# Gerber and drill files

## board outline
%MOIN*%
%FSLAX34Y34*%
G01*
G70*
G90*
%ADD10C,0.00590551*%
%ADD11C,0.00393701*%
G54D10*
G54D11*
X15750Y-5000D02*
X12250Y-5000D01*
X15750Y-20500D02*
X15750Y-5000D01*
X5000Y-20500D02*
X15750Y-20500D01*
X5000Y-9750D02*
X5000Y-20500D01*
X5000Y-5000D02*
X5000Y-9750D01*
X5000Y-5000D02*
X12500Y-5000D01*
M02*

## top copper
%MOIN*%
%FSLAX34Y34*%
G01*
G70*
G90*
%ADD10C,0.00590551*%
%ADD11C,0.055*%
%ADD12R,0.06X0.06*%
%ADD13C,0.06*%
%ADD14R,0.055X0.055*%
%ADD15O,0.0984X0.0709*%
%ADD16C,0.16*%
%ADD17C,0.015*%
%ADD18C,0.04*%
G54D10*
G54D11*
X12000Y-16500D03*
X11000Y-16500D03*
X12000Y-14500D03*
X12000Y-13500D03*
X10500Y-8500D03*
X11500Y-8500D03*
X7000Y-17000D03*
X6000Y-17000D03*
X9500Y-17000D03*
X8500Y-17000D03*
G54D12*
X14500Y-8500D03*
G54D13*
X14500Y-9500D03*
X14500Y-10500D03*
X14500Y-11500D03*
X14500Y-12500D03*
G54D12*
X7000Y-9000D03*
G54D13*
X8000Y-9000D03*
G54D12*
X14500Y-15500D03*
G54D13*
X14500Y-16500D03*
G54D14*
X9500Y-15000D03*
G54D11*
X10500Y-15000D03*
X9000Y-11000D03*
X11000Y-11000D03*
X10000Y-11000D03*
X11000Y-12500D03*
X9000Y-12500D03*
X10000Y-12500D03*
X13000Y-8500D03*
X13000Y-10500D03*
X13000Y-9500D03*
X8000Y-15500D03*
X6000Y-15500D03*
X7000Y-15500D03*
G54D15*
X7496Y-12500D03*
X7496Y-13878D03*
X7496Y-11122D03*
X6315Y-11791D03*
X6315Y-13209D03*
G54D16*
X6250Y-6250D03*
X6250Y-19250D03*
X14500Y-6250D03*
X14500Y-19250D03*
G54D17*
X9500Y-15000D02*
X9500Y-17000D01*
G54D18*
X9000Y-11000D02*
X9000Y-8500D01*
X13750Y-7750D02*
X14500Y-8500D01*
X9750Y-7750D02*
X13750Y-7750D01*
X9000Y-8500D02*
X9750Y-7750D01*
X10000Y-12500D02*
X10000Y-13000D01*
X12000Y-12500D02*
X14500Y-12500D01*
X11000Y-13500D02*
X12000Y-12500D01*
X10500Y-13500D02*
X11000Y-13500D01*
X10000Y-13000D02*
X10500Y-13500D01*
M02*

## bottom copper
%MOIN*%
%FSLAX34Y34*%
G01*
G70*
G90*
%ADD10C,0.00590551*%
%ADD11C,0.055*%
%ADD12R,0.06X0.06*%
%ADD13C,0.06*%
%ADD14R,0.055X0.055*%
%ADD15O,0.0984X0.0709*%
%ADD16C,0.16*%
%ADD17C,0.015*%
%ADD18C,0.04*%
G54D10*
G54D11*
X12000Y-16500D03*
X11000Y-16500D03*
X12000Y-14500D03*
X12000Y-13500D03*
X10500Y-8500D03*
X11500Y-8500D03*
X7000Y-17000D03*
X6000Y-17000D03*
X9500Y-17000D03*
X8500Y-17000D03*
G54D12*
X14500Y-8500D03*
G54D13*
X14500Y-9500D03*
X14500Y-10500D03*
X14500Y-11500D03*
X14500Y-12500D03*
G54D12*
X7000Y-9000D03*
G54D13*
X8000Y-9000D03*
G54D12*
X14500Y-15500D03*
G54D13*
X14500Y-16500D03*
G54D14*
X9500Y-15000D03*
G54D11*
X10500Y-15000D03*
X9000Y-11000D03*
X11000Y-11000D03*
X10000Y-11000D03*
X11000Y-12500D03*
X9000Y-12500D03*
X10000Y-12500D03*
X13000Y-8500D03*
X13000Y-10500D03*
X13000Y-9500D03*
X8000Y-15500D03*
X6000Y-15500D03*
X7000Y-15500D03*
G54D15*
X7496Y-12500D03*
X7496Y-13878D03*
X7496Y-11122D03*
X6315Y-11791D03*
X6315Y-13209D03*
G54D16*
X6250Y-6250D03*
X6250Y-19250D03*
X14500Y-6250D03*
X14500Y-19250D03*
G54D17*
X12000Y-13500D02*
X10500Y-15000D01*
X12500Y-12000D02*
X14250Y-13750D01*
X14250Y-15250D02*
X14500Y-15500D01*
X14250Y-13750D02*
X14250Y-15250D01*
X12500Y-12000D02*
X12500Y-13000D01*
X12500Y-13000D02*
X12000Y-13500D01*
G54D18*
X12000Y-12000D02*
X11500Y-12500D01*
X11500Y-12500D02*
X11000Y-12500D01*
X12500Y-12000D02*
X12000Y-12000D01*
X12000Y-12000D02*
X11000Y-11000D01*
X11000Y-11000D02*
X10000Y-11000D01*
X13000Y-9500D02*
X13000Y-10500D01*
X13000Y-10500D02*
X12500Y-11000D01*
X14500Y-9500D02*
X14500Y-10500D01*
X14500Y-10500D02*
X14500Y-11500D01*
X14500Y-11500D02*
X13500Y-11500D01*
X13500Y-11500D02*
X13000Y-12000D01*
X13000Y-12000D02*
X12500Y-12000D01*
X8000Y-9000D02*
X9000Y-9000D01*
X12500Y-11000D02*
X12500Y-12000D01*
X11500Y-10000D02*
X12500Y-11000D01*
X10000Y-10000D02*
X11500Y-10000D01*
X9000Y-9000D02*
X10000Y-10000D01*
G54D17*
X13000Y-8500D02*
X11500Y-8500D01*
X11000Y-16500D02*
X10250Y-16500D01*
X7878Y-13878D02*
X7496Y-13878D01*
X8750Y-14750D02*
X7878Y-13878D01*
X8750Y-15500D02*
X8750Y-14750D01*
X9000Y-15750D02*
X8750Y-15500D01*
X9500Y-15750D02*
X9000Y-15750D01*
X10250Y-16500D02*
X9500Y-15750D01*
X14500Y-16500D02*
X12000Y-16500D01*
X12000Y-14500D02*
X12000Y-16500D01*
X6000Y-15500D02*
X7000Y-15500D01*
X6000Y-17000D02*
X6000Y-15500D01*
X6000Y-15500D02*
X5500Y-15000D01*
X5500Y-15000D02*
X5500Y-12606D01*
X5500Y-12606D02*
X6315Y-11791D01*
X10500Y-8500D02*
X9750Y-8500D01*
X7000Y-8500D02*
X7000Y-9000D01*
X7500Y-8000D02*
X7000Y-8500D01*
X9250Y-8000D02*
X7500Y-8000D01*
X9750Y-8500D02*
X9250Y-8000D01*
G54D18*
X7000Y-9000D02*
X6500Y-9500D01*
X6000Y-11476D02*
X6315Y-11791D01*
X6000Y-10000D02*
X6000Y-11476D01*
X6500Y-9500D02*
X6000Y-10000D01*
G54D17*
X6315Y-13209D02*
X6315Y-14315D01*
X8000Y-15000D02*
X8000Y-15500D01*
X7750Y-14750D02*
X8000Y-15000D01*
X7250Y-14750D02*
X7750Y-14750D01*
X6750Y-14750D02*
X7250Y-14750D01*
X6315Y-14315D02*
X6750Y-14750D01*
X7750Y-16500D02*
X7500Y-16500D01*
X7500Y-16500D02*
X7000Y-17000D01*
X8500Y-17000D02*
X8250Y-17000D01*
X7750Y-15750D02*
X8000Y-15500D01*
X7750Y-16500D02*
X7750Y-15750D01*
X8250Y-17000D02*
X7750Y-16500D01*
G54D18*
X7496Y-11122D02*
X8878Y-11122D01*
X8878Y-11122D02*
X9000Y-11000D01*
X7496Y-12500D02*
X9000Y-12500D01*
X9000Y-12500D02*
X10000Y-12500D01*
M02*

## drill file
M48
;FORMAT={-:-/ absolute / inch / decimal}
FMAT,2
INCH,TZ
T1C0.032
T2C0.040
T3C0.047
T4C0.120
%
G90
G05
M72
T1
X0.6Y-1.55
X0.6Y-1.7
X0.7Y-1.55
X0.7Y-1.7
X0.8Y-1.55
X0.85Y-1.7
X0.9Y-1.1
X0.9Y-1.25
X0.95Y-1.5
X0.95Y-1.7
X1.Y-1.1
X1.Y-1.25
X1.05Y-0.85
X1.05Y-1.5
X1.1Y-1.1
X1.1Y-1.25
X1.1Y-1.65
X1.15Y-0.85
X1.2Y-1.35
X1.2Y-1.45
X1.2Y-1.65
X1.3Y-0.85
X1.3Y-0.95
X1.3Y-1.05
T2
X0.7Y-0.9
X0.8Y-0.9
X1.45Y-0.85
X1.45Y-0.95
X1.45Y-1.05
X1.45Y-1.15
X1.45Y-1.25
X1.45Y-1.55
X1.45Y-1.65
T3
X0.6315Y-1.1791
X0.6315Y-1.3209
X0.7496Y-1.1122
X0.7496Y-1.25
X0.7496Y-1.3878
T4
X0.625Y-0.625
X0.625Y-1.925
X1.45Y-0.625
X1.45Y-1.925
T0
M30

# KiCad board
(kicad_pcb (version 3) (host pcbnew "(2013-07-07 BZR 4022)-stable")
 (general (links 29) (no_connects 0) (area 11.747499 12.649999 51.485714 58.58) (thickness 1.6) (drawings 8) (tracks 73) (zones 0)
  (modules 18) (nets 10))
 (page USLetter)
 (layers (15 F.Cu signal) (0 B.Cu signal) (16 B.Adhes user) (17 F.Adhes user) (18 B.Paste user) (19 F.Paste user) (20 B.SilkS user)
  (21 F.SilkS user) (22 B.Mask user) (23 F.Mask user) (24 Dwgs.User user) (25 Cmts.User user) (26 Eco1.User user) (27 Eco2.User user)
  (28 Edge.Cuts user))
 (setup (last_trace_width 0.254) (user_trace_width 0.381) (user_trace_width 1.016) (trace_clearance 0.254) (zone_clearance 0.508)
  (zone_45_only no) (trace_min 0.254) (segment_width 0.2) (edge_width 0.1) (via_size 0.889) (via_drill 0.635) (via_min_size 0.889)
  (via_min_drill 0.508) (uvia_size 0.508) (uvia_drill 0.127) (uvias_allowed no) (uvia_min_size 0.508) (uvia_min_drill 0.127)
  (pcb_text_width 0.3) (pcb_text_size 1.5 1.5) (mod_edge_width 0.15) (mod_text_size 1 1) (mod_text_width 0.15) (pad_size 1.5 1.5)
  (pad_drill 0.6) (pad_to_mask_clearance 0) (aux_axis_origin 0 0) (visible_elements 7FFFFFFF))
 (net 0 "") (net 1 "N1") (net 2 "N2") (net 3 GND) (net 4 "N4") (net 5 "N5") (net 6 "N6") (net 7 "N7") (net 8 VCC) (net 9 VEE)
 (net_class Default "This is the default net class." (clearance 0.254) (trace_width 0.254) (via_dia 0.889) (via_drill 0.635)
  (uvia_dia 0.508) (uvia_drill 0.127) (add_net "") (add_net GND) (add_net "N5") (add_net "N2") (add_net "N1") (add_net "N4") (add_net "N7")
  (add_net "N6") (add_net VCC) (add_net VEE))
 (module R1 (layer F.Cu) (at 29.21 41.91 180) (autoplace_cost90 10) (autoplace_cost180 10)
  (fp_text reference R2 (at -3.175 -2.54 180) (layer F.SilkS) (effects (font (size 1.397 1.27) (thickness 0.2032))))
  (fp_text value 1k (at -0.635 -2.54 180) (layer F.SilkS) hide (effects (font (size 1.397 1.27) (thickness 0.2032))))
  (pad 1 thru_hole circle (at -1.27 0 180) (size 1.397 1.397) (drill 0.8128) (layers *.Cu *.Mask F.SilkS) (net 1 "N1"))
  (pad 2 thru_hole circle (at 1.27 0 180) (size 1.397 1.397) (drill 0.8128) (layers *.Cu *.Mask F.SilkS) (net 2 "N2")))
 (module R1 (layer F.Cu) (at 30.48 35.56 90) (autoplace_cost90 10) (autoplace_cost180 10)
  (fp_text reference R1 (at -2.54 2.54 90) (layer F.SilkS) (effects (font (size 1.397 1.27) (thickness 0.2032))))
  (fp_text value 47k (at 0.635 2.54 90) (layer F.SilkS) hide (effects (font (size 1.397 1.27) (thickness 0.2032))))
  (pad 1 thru_hole circle (at -1.27 0 90) (size 1.397 1.397) (drill 0.8128) (layers *.Cu *.Mask F.SilkS) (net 1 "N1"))
  (pad 2 thru_hole circle (at 1.27 0 90) (size 1.397 1.397) (drill 0.8128) (layers *.Cu *.Mask F.SilkS) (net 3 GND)))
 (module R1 (layer F.Cu) (at 27.94 21.59) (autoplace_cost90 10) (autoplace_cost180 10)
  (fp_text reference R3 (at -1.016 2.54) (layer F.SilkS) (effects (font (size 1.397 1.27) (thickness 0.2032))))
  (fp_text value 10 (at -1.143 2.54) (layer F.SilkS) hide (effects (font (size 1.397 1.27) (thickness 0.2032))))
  (pad 1 thru_hole circle (at -1.27 0) (size 1.397 1.397) (drill 0.8128) (layers *.Cu *.Mask F.SilkS) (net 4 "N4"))
  (pad 2 thru_hole circle (at 1.27 0) (size 1.397 1.397) (drill 0.8128) (layers *.Cu *.Mask F.SilkS) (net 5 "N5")))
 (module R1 (layer F.Cu) (at 16.51 43.18 180) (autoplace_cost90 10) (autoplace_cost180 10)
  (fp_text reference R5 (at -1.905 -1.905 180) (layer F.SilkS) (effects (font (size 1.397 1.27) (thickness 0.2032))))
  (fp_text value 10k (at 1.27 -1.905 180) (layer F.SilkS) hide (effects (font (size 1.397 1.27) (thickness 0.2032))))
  (pad 1 thru_hole circle (at -1.27 0 180) (size 1.397 1.397) (drill 0.8128) (layers *.Cu *.Mask F.SilkS) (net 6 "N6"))
  (pad 2 thru_hole circle (at 1.27 0 180) (size 1.397 1.397) (drill 0.8128) (layers *.Cu *.Mask F.SilkS) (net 4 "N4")))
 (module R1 (layer F.Cu) (at 22.86 43.18 180) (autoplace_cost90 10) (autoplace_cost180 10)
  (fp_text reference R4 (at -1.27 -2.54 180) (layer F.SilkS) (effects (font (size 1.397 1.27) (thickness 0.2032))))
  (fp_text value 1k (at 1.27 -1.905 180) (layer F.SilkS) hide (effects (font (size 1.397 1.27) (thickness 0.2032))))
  (pad 1 thru_hole circle (at -1.27 0 180) (size 1.397 1.397) (drill 0.8128) (layers *.Cu *.Mask F.SilkS) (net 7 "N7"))
  (pad 2 thru_hole circle (at 1.27 0 180) (size 1.397 1.397) (drill 0.8128) (layers *.Cu *.Mask F.SilkS) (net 6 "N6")))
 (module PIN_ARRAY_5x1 (layer F.Cu) (at 36.83 26.67 270)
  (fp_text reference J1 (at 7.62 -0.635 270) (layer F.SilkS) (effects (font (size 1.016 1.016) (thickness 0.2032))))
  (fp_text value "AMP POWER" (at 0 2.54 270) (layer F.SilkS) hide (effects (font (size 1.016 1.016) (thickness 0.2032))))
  (pad 1 thru_hole rect (at -5.08 0 270) (size 1.524 1.524) (drill 1.016) (layers *.Cu *.Mask F.SilkS) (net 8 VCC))
  (pad 2 thru_hole circle (at -2.54 0 270) (size 1.524 1.524) (drill 1.016) (layers *.Cu *.Mask F.SilkS) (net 3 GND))
  (pad 3 thru_hole circle (at 0 0 270) (size 1.524 1.524) (drill 1.016) (layers *.Cu *.Mask F.SilkS) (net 3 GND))
  (pad 4 thru_hole circle (at 2.54 0 270) (size 1.524 1.524) (drill 1.016) (layers *.Cu *.Mask F.SilkS) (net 3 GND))
  (pad 5 thru_hole circle (at 5.08 0 270) (size 1.524 1.524) (drill 1.016) (layers *.Cu *.Mask F.SilkS) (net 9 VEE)))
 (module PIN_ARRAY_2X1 (layer F.Cu) (at 19.05 22.86)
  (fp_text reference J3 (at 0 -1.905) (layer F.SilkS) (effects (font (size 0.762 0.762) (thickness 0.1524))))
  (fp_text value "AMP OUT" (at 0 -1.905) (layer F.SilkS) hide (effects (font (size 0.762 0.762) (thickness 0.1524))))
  (pad 1 thru_hole rect (at -1.27 0) (size 1.524 1.524) (drill 1.016) (layers *.Cu *.Mask F.SilkS) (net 4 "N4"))
  (pad 2 thru_hole circle (at 1.27 0) (size 1.524 1.524) (drill 1.016) (layers *.Cu *.Mask F.SilkS) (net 3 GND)))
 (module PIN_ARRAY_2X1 (layer F.Cu) (at 36.83 40.64 270)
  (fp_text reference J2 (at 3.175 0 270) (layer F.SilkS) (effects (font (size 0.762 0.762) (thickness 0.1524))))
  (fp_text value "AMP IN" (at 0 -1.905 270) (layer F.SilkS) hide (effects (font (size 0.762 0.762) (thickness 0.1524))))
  (pad 1 thru_hole rect (at -1.27 0 270) (size 1.524 1.524) (drill 1.016) (layers *.Cu *.Mask F.SilkS) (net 3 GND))
  (pad 2 thru_hole circle (at 1.27 0 270) (size 1.524 1.524) (drill 1.016) (layers *.Cu *.Mask F.SilkS) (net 1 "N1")))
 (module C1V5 (layer F.Cu) (at 25.4 38.1)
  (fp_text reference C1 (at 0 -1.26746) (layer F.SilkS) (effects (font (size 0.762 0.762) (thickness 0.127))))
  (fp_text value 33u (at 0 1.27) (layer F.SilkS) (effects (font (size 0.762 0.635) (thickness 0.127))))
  (pad 1 thru_hole rect (at -1.27 0) (size 1.397 1.397) (drill 0.8128) (layers *.Cu *.Mask F.SilkS) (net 7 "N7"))
  (pad 2 thru_hole circle (at 1.27 0) (size 1.397 1.397) (drill 0.8128) (layers *.Cu *.Mask F.SilkS) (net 3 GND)))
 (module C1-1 (layer F.Cu) (at 25.4 27.94)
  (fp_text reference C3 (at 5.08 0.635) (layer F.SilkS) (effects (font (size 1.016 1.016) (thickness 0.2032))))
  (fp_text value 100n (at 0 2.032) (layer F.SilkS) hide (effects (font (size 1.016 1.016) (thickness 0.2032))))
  (pad 1 thru_hole circle (at -2.54 0) (size 1.397 1.397) (drill 0.8128) (layers *.Cu *.Mask F.SilkS) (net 8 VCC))
  (pad 2 thru_hole circle (at 2.54 0) (size 1.397 1.397) (drill 0.8128) (layers *.Cu *.Mask F.SilkS) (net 3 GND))
  (pad 2 thru_hole circle (at 0 0) (size 1.397 1.397) (drill 0.8128) (layers *.Cu *.Mask F.SilkS) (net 3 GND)))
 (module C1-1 (layer F.Cu) (at 25.4 31.75 180)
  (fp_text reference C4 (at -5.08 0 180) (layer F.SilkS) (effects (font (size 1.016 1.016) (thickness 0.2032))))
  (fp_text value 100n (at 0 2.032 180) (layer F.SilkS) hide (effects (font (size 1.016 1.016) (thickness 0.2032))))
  (pad 1 thru_hole circle (at -2.54 0 180) (size 1.397 1.397) (drill 0.8128) (layers *.Cu *.Mask F.SilkS) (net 3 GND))
  (pad 2 thru_hole circle (at 2.54 0 180) (size 1.397 1.397) (drill 0.8128) (layers *.Cu *.Mask F.SilkS) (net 9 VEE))
  (pad 2 thru_hole circle (at 0 0 180) (size 1.397 1.397) (drill 0.8128) (layers *.Cu *.Mask F.SilkS) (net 9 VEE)))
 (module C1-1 (layer F.Cu) (at 33.02 24.13 270)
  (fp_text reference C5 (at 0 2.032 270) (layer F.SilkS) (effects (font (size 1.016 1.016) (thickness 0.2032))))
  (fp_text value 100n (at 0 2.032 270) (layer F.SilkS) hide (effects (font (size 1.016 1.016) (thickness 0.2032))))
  (pad 1 thru_hole circle (at -2.54 0 270) (size 1.397 1.397) (drill 0.8128) (layers *.Cu *.Mask F.SilkS) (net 5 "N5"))
  (pad 2 thru_hole circle (at 2.54 0 270) (size 1.397 1.397) (drill 0.8128) (layers *.Cu *.Mask F.SilkS) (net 3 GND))
  (pad 2 thru_hole circle (at 0 0 270) (size 1.397 1.397) (drill 0.8128) (layers *.Cu *.Mask F.SilkS) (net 3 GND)))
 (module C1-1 (layer F.Cu) (at 17.78 39.37 180)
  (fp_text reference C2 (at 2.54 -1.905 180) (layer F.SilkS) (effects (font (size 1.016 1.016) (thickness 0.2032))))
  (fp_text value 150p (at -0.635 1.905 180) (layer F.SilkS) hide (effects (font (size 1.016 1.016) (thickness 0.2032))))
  (pad 1 thru_hole circle (at -2.54 0 180) (size 1.397 1.397) (drill 0.8128) (layers *.Cu *.Mask F.SilkS) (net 6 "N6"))
  (pad 2 thru_hole circle (at 2.54 0 180) (size 1.397 1.397) (drill 0.8128) (layers *.Cu *.Mask F.SilkS) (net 4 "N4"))
  (pad 2 thru_hole circle (at 0 0 180) (size 1.397 1.397) (drill 0.8128) (layers *.Cu *.Mask F.SilkS) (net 4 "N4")))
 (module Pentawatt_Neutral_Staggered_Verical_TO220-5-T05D (layer F.Cu) (at 15.24 31.75 90)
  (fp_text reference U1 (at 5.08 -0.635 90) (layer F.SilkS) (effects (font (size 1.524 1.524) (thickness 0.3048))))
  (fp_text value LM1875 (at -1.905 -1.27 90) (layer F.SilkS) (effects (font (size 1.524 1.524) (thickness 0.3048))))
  (pad 3 thru_hole oval (at 0 3.79984 180) (size 2.49936 1.80086) (drill 1.19888) (layers *.Cu *.Mask F.SilkS) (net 9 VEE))
  (pad 1 thru_hole oval (at -3.50012 3.79984 180) (size 2.49936 1.80086) (drill 1.19888) (layers *.Cu *.Mask F.SilkS) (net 2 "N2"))
  (pad 5 thru_hole oval (at 3.50012 3.79984 180) (size 2.49936 1.80086) (drill 1.19888) (layers *.Cu *.Mask F.SilkS) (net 8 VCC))
  (pad 4 thru_hole oval (at 1.80086 0.8001 180) (size 2.49936 1.80086) (drill 1.19888) (layers *.Cu *.Mask F.SilkS) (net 4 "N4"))
  (pad 2 thru_hole oval (at -1.80086 0.8001 180) (size 2.49936 1.80086) (drill 1.19888) (layers *.Cu *.Mask F.SilkS) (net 6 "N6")))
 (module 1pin (layer F.Cu) (at 15.875 15.875)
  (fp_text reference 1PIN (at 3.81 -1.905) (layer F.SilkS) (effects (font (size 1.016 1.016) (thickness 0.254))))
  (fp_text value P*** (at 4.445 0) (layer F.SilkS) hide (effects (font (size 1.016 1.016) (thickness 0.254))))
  (pad 1 thru_hole circle (at 0 0) (size 4.064 4.064) (drill 3.048) (layers *.Cu *.Mask F.SilkS)))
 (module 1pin (layer F.Cu) (at 15.875 48.895)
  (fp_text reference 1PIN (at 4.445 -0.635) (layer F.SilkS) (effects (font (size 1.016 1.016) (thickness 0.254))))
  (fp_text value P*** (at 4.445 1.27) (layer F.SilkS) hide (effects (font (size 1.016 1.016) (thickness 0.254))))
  (pad 1 thru_hole circle (at 0 0) (size 4.064 4.064) (drill 3.048) (layers *.Cu *.Mask F.SilkS)))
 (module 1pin (layer F.Cu) (at 36.83 15.875)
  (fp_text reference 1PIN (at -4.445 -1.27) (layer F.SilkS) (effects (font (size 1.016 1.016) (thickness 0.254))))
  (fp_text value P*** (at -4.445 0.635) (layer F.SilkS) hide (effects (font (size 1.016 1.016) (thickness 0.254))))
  (pad 1 thru_hole circle (at 0 0) (size 4.064 4.064) (drill 3.048) (layers *.Cu *.Mask F.SilkS)))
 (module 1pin (layer F.Cu) (at 36.83 48.895)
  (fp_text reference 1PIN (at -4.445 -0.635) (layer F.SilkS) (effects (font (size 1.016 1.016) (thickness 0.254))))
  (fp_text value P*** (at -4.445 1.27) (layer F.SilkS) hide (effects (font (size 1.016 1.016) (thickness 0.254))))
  (pad 1 thru_hole circle (at 0 0) (size 4.064 4.064) (drill 3.048) (layers *.Cu *.Mask F.SilkS)))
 (gr_line (start 40.005 12.7) (end 31.115 12.7) (angle 90) (layer Edge.Cuts) (width 0.1))
 (gr_line (start 40.005 52.07) (end 40.005 12.7) (angle 90) (layer Edge.Cuts) (width 0.1))
 (gr_line (start 12.7 52.07) (end 40.005 52.07) (angle 90) (layer Edge.Cuts) (width 0.1))
 (gr_line (start 12.7 24.765) (end 12.7 52.07) (angle 90) (layer Edge.Cuts) (width 0.1))
 (gr_line (start 12.7 12.7) (end 12.7 24.765) (angle 90) (layer Edge.Cuts) (width 0.1))
 (gr_line (start 12.7 12.7) (end 31.75 12.7) (angle 90) (layer Edge.Cuts) (width 0.1))
 (segment (start 30.48 34.29) (end 26.67 38.1) (width 0.381) (layer B.Cu) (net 3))
 (segment (start 31.75 30.48) (end 36.195 34.925) (width 0.381) (layer B.Cu) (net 3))
 (segment (start 36.195 38.735) (end 36.83 39.37) (width 0.381) (layer B.Cu) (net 3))
 (segment (start 36.195 34.925) (end 36.195 38.735) (width 0.381) (layer B.Cu) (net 3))
 (segment (start 31.75 30.48) (end 31.75 33.02) (width 0.381) (layer B.Cu) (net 3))
 (segment (start 31.75 33.02) (end 30.48 34.29) (width 0.381) (layer B.Cu) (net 3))
 (segment (start 30.48 30.48) (end 29.21 31.75) (width 1.016) (layer B.Cu) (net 3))
 (segment (start 29.21 31.75) (end 27.94 31.75) (width 1.016) (layer B.Cu) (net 3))
 (segment (start 31.75 30.48) (end 30.48 30.48) (width 1.016) (layer B.Cu) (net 3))
 (segment (start 30.48 30.48) (end 27.94 27.94) (width 1.016) (layer B.Cu) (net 3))
 (segment (start 27.94 27.94) (end 25.4 27.94) (width 1.016) (layer B.Cu) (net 3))
 (segment (start 33.02 24.13) (end 33.02 26.67) (width 1.016) (layer B.Cu) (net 3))
 (segment (start 33.02 26.67) (end 31.75 27.94) (width 1.016) (layer B.Cu) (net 3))
 (segment (start 36.83 24.13) (end 36.83 26.67) (width 1.016) (layer B.Cu) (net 3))
 (segment (start 36.83 26.67) (end 36.83 29.21) (width 1.016) (layer B.Cu) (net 3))
 (segment (start 36.83 29.21) (end 34.29 29.21) (width 1.016) (layer B.Cu) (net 3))
 (segment (start 34.29 29.21) (end 33.02 30.48) (width 1.016) (layer B.Cu) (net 3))
 (segment (start 33.02 30.48) (end 31.75 30.48) (width 1.016) (layer B.Cu) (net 3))
 (segment (start 20.32 22.86) (end 22.86 22.86) (width 1.016) (layer B.Cu) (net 3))
 (segment (start 31.75 27.94) (end 31.75 30.48) (width 1.016) (layer B.Cu) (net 3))
 (segment (start 29.21 25.4) (end 31.75 27.94) (width 1.016) (layer B.Cu) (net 3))
 (segment (start 25.4 25.4) (end 29.21 25.4) (width 1.016) (layer B.Cu) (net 3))
 (segment (start 22.86 22.86) (end 25.4 25.4) (width 1.016) (layer B.Cu) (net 3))
 (segment (start 33.02 21.59) (end 29.21 21.59) (width 0.381) (layer B.Cu) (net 5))
 (segment (start 27.94 41.91) (end 26.035 41.91) (width 0.381) (layer B.Cu) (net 2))
 (segment (start 20.01012 35.25012) (end 19.03984 35.25012) (width 0.381) (layer B.Cu) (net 2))
 (segment (start 22.225 37.465) (end 20.01012 35.25012) (width 0.381) (layer B.Cu) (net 2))
 (segment (start 22.225 39.37) (end 22.225 37.465) (width 0.381) (layer B.Cu) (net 2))
 (segment (start 22.86 40.005) (end 22.225 39.37) (width 0.381) (layer B.Cu) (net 2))
 (segment (start 24.13 40.005) (end 22.86 40.005) (width 0.381) (layer B.Cu) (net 2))
 (segment (start 26.035 41.91) (end 24.13 40.005) (width 0.381) (layer B.Cu) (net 2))
 (segment (start 36.83 41.91) (end 30.48 41.91) (width 0.381) (layer B.Cu) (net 1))
 (segment (start 30.48 36.83) (end 30.48 41.91) (width 0.381) (layer B.Cu) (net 1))
 (segment (start 15.24 39.37) (end 17.78 39.37) (width 0.381) (layer B.Cu) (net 4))
 (segment (start 15.24 43.18) (end 15.24 39.37) (width 0.381) (layer B.Cu) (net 4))
 (segment (start 15.24 39.37) (end 13.97 38.1) (width 0.381) (layer B.Cu) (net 4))
 (segment (start 13.97 38.1) (end 13.97 32.01924) (width 0.381) (layer B.Cu) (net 4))
 (segment (start 13.97 32.01924) (end 16.0401 29.94914) (width 0.381) (layer B.Cu) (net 4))
 (segment (start 26.67 21.59) (end 24.765 21.59) (width 0.381) (layer B.Cu) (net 4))
 (segment (start 17.78 21.59) (end 17.78 22.86) (width 0.381) (layer B.Cu) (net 4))
 (segment (start 19.05 20.32) (end 17.78 21.59) (width 0.381) (layer B.Cu) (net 4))
 (segment (start 23.495 20.32) (end 19.05 20.32) (width 0.381) (layer B.Cu) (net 4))
 (segment (start 24.765 21.59) (end 23.495 20.32) (width 0.381) (layer B.Cu) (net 4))
 (segment (start 17.78 22.86) (end 16.51 24.13) (width 1.016) (layer B.Cu) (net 4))
 (segment (start 15.24 29.14904) (end 16.0401 29.94914) (width 1.016) (layer B.Cu) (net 4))
 (segment (start 15.24 25.4) (end 15.24 29.14904) (width 1.016) (layer B.Cu) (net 4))
 (segment (start 16.51 24.13) (end 15.24 25.4) (width 1.016) (layer B.Cu) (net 4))
 (segment (start 24.13 38.1) (end 24.13 43.18) (width 0.381) (layer F.Cu) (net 7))
 (segment (start 16.0401 33.55086) (end 16.0401 36.3601) (width 0.381) (layer B.Cu) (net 6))
 (segment (start 20.32 38.1) (end 20.32 39.37) (width 0.381) (layer B.Cu) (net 6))
 (segment (start 19.685 37.465) (end 20.32 38.1) (width 0.381) (layer B.Cu) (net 6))
 (segment (start 18.415 37.465) (end 19.685 37.465) (width 0.381) (layer B.Cu) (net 6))
 (segment (start 17.145 37.465) (end 18.415 37.465) (width 0.381) (layer B.Cu) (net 6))
 (segment (start 16.0401 36.3601) (end 17.145 37.465) (width 0.381) (layer B.Cu) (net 6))
 (segment (start 19.685 41.91) (end 19.05 41.91) (width 0.381) (layer B.Cu) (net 6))
 (segment (start 19.05 41.91) (end 17.78 43.18) (width 0.381) (layer B.Cu) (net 6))
 (segment (start 21.59 43.18) (end 20.955 43.18) (width 0.381) (layer B.Cu) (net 6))
 (segment (start 19.685 40.005) (end 20.32 39.37) (width 0.381) (layer B.Cu) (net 6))
 (segment (start 19.685 41.91) (end 19.685 40.005) (width 0.381) (layer B.Cu) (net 6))
 (segment (start 20.955 43.18) (end 19.685 41.91) (width 0.381) (layer B.Cu) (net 6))
 (segment (start 22.86 27.94) (end 22.86 21.59) (width 1.016) (layer F.Cu) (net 8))
 (segment (start 34.925 19.685) (end 36.83 21.59) (width 1.016) (layer F.Cu) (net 8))
 (segment (start 24.765 19.685) (end 34.925 19.685) (width 1.016) (layer F.Cu) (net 8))
 (segment (start 22.86 21.59) (end 24.765 19.685) (width 1.016) (layer F.Cu) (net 8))
 (segment (start 19.03984 28.24988) (end 22.55012 28.24988) (width 1.016) (layer B.Cu) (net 8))
 (segment (start 22.55012 28.24988) (end 22.86 27.94) (width 1.016) (layer B.Cu) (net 8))
 (segment (start 25.4 31.75) (end 25.4 33.02) (width 1.016) (layer F.Cu) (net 9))
 (segment (start 30.48 31.75) (end 36.83 31.75) (width 1.016) (layer F.Cu) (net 9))
 (segment (start 27.94 34.29) (end 30.48 31.75) (width 1.016) (layer F.Cu) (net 9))
 (segment (start 26.67 34.29) (end 27.94 34.29) (width 1.016) (layer F.Cu) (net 9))
 (segment (start 25.4 33.02) (end 26.67 34.29) (width 1.016) (layer F.Cu) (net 9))
 (segment (start 19.03984 31.75) (end 22.86 31.75) (width 1.016) (layer B.Cu) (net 9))
 (segment (start 22.86 31.75) (end 25.4 31.75) (width 1.016) (layer B.Cu) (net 9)))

